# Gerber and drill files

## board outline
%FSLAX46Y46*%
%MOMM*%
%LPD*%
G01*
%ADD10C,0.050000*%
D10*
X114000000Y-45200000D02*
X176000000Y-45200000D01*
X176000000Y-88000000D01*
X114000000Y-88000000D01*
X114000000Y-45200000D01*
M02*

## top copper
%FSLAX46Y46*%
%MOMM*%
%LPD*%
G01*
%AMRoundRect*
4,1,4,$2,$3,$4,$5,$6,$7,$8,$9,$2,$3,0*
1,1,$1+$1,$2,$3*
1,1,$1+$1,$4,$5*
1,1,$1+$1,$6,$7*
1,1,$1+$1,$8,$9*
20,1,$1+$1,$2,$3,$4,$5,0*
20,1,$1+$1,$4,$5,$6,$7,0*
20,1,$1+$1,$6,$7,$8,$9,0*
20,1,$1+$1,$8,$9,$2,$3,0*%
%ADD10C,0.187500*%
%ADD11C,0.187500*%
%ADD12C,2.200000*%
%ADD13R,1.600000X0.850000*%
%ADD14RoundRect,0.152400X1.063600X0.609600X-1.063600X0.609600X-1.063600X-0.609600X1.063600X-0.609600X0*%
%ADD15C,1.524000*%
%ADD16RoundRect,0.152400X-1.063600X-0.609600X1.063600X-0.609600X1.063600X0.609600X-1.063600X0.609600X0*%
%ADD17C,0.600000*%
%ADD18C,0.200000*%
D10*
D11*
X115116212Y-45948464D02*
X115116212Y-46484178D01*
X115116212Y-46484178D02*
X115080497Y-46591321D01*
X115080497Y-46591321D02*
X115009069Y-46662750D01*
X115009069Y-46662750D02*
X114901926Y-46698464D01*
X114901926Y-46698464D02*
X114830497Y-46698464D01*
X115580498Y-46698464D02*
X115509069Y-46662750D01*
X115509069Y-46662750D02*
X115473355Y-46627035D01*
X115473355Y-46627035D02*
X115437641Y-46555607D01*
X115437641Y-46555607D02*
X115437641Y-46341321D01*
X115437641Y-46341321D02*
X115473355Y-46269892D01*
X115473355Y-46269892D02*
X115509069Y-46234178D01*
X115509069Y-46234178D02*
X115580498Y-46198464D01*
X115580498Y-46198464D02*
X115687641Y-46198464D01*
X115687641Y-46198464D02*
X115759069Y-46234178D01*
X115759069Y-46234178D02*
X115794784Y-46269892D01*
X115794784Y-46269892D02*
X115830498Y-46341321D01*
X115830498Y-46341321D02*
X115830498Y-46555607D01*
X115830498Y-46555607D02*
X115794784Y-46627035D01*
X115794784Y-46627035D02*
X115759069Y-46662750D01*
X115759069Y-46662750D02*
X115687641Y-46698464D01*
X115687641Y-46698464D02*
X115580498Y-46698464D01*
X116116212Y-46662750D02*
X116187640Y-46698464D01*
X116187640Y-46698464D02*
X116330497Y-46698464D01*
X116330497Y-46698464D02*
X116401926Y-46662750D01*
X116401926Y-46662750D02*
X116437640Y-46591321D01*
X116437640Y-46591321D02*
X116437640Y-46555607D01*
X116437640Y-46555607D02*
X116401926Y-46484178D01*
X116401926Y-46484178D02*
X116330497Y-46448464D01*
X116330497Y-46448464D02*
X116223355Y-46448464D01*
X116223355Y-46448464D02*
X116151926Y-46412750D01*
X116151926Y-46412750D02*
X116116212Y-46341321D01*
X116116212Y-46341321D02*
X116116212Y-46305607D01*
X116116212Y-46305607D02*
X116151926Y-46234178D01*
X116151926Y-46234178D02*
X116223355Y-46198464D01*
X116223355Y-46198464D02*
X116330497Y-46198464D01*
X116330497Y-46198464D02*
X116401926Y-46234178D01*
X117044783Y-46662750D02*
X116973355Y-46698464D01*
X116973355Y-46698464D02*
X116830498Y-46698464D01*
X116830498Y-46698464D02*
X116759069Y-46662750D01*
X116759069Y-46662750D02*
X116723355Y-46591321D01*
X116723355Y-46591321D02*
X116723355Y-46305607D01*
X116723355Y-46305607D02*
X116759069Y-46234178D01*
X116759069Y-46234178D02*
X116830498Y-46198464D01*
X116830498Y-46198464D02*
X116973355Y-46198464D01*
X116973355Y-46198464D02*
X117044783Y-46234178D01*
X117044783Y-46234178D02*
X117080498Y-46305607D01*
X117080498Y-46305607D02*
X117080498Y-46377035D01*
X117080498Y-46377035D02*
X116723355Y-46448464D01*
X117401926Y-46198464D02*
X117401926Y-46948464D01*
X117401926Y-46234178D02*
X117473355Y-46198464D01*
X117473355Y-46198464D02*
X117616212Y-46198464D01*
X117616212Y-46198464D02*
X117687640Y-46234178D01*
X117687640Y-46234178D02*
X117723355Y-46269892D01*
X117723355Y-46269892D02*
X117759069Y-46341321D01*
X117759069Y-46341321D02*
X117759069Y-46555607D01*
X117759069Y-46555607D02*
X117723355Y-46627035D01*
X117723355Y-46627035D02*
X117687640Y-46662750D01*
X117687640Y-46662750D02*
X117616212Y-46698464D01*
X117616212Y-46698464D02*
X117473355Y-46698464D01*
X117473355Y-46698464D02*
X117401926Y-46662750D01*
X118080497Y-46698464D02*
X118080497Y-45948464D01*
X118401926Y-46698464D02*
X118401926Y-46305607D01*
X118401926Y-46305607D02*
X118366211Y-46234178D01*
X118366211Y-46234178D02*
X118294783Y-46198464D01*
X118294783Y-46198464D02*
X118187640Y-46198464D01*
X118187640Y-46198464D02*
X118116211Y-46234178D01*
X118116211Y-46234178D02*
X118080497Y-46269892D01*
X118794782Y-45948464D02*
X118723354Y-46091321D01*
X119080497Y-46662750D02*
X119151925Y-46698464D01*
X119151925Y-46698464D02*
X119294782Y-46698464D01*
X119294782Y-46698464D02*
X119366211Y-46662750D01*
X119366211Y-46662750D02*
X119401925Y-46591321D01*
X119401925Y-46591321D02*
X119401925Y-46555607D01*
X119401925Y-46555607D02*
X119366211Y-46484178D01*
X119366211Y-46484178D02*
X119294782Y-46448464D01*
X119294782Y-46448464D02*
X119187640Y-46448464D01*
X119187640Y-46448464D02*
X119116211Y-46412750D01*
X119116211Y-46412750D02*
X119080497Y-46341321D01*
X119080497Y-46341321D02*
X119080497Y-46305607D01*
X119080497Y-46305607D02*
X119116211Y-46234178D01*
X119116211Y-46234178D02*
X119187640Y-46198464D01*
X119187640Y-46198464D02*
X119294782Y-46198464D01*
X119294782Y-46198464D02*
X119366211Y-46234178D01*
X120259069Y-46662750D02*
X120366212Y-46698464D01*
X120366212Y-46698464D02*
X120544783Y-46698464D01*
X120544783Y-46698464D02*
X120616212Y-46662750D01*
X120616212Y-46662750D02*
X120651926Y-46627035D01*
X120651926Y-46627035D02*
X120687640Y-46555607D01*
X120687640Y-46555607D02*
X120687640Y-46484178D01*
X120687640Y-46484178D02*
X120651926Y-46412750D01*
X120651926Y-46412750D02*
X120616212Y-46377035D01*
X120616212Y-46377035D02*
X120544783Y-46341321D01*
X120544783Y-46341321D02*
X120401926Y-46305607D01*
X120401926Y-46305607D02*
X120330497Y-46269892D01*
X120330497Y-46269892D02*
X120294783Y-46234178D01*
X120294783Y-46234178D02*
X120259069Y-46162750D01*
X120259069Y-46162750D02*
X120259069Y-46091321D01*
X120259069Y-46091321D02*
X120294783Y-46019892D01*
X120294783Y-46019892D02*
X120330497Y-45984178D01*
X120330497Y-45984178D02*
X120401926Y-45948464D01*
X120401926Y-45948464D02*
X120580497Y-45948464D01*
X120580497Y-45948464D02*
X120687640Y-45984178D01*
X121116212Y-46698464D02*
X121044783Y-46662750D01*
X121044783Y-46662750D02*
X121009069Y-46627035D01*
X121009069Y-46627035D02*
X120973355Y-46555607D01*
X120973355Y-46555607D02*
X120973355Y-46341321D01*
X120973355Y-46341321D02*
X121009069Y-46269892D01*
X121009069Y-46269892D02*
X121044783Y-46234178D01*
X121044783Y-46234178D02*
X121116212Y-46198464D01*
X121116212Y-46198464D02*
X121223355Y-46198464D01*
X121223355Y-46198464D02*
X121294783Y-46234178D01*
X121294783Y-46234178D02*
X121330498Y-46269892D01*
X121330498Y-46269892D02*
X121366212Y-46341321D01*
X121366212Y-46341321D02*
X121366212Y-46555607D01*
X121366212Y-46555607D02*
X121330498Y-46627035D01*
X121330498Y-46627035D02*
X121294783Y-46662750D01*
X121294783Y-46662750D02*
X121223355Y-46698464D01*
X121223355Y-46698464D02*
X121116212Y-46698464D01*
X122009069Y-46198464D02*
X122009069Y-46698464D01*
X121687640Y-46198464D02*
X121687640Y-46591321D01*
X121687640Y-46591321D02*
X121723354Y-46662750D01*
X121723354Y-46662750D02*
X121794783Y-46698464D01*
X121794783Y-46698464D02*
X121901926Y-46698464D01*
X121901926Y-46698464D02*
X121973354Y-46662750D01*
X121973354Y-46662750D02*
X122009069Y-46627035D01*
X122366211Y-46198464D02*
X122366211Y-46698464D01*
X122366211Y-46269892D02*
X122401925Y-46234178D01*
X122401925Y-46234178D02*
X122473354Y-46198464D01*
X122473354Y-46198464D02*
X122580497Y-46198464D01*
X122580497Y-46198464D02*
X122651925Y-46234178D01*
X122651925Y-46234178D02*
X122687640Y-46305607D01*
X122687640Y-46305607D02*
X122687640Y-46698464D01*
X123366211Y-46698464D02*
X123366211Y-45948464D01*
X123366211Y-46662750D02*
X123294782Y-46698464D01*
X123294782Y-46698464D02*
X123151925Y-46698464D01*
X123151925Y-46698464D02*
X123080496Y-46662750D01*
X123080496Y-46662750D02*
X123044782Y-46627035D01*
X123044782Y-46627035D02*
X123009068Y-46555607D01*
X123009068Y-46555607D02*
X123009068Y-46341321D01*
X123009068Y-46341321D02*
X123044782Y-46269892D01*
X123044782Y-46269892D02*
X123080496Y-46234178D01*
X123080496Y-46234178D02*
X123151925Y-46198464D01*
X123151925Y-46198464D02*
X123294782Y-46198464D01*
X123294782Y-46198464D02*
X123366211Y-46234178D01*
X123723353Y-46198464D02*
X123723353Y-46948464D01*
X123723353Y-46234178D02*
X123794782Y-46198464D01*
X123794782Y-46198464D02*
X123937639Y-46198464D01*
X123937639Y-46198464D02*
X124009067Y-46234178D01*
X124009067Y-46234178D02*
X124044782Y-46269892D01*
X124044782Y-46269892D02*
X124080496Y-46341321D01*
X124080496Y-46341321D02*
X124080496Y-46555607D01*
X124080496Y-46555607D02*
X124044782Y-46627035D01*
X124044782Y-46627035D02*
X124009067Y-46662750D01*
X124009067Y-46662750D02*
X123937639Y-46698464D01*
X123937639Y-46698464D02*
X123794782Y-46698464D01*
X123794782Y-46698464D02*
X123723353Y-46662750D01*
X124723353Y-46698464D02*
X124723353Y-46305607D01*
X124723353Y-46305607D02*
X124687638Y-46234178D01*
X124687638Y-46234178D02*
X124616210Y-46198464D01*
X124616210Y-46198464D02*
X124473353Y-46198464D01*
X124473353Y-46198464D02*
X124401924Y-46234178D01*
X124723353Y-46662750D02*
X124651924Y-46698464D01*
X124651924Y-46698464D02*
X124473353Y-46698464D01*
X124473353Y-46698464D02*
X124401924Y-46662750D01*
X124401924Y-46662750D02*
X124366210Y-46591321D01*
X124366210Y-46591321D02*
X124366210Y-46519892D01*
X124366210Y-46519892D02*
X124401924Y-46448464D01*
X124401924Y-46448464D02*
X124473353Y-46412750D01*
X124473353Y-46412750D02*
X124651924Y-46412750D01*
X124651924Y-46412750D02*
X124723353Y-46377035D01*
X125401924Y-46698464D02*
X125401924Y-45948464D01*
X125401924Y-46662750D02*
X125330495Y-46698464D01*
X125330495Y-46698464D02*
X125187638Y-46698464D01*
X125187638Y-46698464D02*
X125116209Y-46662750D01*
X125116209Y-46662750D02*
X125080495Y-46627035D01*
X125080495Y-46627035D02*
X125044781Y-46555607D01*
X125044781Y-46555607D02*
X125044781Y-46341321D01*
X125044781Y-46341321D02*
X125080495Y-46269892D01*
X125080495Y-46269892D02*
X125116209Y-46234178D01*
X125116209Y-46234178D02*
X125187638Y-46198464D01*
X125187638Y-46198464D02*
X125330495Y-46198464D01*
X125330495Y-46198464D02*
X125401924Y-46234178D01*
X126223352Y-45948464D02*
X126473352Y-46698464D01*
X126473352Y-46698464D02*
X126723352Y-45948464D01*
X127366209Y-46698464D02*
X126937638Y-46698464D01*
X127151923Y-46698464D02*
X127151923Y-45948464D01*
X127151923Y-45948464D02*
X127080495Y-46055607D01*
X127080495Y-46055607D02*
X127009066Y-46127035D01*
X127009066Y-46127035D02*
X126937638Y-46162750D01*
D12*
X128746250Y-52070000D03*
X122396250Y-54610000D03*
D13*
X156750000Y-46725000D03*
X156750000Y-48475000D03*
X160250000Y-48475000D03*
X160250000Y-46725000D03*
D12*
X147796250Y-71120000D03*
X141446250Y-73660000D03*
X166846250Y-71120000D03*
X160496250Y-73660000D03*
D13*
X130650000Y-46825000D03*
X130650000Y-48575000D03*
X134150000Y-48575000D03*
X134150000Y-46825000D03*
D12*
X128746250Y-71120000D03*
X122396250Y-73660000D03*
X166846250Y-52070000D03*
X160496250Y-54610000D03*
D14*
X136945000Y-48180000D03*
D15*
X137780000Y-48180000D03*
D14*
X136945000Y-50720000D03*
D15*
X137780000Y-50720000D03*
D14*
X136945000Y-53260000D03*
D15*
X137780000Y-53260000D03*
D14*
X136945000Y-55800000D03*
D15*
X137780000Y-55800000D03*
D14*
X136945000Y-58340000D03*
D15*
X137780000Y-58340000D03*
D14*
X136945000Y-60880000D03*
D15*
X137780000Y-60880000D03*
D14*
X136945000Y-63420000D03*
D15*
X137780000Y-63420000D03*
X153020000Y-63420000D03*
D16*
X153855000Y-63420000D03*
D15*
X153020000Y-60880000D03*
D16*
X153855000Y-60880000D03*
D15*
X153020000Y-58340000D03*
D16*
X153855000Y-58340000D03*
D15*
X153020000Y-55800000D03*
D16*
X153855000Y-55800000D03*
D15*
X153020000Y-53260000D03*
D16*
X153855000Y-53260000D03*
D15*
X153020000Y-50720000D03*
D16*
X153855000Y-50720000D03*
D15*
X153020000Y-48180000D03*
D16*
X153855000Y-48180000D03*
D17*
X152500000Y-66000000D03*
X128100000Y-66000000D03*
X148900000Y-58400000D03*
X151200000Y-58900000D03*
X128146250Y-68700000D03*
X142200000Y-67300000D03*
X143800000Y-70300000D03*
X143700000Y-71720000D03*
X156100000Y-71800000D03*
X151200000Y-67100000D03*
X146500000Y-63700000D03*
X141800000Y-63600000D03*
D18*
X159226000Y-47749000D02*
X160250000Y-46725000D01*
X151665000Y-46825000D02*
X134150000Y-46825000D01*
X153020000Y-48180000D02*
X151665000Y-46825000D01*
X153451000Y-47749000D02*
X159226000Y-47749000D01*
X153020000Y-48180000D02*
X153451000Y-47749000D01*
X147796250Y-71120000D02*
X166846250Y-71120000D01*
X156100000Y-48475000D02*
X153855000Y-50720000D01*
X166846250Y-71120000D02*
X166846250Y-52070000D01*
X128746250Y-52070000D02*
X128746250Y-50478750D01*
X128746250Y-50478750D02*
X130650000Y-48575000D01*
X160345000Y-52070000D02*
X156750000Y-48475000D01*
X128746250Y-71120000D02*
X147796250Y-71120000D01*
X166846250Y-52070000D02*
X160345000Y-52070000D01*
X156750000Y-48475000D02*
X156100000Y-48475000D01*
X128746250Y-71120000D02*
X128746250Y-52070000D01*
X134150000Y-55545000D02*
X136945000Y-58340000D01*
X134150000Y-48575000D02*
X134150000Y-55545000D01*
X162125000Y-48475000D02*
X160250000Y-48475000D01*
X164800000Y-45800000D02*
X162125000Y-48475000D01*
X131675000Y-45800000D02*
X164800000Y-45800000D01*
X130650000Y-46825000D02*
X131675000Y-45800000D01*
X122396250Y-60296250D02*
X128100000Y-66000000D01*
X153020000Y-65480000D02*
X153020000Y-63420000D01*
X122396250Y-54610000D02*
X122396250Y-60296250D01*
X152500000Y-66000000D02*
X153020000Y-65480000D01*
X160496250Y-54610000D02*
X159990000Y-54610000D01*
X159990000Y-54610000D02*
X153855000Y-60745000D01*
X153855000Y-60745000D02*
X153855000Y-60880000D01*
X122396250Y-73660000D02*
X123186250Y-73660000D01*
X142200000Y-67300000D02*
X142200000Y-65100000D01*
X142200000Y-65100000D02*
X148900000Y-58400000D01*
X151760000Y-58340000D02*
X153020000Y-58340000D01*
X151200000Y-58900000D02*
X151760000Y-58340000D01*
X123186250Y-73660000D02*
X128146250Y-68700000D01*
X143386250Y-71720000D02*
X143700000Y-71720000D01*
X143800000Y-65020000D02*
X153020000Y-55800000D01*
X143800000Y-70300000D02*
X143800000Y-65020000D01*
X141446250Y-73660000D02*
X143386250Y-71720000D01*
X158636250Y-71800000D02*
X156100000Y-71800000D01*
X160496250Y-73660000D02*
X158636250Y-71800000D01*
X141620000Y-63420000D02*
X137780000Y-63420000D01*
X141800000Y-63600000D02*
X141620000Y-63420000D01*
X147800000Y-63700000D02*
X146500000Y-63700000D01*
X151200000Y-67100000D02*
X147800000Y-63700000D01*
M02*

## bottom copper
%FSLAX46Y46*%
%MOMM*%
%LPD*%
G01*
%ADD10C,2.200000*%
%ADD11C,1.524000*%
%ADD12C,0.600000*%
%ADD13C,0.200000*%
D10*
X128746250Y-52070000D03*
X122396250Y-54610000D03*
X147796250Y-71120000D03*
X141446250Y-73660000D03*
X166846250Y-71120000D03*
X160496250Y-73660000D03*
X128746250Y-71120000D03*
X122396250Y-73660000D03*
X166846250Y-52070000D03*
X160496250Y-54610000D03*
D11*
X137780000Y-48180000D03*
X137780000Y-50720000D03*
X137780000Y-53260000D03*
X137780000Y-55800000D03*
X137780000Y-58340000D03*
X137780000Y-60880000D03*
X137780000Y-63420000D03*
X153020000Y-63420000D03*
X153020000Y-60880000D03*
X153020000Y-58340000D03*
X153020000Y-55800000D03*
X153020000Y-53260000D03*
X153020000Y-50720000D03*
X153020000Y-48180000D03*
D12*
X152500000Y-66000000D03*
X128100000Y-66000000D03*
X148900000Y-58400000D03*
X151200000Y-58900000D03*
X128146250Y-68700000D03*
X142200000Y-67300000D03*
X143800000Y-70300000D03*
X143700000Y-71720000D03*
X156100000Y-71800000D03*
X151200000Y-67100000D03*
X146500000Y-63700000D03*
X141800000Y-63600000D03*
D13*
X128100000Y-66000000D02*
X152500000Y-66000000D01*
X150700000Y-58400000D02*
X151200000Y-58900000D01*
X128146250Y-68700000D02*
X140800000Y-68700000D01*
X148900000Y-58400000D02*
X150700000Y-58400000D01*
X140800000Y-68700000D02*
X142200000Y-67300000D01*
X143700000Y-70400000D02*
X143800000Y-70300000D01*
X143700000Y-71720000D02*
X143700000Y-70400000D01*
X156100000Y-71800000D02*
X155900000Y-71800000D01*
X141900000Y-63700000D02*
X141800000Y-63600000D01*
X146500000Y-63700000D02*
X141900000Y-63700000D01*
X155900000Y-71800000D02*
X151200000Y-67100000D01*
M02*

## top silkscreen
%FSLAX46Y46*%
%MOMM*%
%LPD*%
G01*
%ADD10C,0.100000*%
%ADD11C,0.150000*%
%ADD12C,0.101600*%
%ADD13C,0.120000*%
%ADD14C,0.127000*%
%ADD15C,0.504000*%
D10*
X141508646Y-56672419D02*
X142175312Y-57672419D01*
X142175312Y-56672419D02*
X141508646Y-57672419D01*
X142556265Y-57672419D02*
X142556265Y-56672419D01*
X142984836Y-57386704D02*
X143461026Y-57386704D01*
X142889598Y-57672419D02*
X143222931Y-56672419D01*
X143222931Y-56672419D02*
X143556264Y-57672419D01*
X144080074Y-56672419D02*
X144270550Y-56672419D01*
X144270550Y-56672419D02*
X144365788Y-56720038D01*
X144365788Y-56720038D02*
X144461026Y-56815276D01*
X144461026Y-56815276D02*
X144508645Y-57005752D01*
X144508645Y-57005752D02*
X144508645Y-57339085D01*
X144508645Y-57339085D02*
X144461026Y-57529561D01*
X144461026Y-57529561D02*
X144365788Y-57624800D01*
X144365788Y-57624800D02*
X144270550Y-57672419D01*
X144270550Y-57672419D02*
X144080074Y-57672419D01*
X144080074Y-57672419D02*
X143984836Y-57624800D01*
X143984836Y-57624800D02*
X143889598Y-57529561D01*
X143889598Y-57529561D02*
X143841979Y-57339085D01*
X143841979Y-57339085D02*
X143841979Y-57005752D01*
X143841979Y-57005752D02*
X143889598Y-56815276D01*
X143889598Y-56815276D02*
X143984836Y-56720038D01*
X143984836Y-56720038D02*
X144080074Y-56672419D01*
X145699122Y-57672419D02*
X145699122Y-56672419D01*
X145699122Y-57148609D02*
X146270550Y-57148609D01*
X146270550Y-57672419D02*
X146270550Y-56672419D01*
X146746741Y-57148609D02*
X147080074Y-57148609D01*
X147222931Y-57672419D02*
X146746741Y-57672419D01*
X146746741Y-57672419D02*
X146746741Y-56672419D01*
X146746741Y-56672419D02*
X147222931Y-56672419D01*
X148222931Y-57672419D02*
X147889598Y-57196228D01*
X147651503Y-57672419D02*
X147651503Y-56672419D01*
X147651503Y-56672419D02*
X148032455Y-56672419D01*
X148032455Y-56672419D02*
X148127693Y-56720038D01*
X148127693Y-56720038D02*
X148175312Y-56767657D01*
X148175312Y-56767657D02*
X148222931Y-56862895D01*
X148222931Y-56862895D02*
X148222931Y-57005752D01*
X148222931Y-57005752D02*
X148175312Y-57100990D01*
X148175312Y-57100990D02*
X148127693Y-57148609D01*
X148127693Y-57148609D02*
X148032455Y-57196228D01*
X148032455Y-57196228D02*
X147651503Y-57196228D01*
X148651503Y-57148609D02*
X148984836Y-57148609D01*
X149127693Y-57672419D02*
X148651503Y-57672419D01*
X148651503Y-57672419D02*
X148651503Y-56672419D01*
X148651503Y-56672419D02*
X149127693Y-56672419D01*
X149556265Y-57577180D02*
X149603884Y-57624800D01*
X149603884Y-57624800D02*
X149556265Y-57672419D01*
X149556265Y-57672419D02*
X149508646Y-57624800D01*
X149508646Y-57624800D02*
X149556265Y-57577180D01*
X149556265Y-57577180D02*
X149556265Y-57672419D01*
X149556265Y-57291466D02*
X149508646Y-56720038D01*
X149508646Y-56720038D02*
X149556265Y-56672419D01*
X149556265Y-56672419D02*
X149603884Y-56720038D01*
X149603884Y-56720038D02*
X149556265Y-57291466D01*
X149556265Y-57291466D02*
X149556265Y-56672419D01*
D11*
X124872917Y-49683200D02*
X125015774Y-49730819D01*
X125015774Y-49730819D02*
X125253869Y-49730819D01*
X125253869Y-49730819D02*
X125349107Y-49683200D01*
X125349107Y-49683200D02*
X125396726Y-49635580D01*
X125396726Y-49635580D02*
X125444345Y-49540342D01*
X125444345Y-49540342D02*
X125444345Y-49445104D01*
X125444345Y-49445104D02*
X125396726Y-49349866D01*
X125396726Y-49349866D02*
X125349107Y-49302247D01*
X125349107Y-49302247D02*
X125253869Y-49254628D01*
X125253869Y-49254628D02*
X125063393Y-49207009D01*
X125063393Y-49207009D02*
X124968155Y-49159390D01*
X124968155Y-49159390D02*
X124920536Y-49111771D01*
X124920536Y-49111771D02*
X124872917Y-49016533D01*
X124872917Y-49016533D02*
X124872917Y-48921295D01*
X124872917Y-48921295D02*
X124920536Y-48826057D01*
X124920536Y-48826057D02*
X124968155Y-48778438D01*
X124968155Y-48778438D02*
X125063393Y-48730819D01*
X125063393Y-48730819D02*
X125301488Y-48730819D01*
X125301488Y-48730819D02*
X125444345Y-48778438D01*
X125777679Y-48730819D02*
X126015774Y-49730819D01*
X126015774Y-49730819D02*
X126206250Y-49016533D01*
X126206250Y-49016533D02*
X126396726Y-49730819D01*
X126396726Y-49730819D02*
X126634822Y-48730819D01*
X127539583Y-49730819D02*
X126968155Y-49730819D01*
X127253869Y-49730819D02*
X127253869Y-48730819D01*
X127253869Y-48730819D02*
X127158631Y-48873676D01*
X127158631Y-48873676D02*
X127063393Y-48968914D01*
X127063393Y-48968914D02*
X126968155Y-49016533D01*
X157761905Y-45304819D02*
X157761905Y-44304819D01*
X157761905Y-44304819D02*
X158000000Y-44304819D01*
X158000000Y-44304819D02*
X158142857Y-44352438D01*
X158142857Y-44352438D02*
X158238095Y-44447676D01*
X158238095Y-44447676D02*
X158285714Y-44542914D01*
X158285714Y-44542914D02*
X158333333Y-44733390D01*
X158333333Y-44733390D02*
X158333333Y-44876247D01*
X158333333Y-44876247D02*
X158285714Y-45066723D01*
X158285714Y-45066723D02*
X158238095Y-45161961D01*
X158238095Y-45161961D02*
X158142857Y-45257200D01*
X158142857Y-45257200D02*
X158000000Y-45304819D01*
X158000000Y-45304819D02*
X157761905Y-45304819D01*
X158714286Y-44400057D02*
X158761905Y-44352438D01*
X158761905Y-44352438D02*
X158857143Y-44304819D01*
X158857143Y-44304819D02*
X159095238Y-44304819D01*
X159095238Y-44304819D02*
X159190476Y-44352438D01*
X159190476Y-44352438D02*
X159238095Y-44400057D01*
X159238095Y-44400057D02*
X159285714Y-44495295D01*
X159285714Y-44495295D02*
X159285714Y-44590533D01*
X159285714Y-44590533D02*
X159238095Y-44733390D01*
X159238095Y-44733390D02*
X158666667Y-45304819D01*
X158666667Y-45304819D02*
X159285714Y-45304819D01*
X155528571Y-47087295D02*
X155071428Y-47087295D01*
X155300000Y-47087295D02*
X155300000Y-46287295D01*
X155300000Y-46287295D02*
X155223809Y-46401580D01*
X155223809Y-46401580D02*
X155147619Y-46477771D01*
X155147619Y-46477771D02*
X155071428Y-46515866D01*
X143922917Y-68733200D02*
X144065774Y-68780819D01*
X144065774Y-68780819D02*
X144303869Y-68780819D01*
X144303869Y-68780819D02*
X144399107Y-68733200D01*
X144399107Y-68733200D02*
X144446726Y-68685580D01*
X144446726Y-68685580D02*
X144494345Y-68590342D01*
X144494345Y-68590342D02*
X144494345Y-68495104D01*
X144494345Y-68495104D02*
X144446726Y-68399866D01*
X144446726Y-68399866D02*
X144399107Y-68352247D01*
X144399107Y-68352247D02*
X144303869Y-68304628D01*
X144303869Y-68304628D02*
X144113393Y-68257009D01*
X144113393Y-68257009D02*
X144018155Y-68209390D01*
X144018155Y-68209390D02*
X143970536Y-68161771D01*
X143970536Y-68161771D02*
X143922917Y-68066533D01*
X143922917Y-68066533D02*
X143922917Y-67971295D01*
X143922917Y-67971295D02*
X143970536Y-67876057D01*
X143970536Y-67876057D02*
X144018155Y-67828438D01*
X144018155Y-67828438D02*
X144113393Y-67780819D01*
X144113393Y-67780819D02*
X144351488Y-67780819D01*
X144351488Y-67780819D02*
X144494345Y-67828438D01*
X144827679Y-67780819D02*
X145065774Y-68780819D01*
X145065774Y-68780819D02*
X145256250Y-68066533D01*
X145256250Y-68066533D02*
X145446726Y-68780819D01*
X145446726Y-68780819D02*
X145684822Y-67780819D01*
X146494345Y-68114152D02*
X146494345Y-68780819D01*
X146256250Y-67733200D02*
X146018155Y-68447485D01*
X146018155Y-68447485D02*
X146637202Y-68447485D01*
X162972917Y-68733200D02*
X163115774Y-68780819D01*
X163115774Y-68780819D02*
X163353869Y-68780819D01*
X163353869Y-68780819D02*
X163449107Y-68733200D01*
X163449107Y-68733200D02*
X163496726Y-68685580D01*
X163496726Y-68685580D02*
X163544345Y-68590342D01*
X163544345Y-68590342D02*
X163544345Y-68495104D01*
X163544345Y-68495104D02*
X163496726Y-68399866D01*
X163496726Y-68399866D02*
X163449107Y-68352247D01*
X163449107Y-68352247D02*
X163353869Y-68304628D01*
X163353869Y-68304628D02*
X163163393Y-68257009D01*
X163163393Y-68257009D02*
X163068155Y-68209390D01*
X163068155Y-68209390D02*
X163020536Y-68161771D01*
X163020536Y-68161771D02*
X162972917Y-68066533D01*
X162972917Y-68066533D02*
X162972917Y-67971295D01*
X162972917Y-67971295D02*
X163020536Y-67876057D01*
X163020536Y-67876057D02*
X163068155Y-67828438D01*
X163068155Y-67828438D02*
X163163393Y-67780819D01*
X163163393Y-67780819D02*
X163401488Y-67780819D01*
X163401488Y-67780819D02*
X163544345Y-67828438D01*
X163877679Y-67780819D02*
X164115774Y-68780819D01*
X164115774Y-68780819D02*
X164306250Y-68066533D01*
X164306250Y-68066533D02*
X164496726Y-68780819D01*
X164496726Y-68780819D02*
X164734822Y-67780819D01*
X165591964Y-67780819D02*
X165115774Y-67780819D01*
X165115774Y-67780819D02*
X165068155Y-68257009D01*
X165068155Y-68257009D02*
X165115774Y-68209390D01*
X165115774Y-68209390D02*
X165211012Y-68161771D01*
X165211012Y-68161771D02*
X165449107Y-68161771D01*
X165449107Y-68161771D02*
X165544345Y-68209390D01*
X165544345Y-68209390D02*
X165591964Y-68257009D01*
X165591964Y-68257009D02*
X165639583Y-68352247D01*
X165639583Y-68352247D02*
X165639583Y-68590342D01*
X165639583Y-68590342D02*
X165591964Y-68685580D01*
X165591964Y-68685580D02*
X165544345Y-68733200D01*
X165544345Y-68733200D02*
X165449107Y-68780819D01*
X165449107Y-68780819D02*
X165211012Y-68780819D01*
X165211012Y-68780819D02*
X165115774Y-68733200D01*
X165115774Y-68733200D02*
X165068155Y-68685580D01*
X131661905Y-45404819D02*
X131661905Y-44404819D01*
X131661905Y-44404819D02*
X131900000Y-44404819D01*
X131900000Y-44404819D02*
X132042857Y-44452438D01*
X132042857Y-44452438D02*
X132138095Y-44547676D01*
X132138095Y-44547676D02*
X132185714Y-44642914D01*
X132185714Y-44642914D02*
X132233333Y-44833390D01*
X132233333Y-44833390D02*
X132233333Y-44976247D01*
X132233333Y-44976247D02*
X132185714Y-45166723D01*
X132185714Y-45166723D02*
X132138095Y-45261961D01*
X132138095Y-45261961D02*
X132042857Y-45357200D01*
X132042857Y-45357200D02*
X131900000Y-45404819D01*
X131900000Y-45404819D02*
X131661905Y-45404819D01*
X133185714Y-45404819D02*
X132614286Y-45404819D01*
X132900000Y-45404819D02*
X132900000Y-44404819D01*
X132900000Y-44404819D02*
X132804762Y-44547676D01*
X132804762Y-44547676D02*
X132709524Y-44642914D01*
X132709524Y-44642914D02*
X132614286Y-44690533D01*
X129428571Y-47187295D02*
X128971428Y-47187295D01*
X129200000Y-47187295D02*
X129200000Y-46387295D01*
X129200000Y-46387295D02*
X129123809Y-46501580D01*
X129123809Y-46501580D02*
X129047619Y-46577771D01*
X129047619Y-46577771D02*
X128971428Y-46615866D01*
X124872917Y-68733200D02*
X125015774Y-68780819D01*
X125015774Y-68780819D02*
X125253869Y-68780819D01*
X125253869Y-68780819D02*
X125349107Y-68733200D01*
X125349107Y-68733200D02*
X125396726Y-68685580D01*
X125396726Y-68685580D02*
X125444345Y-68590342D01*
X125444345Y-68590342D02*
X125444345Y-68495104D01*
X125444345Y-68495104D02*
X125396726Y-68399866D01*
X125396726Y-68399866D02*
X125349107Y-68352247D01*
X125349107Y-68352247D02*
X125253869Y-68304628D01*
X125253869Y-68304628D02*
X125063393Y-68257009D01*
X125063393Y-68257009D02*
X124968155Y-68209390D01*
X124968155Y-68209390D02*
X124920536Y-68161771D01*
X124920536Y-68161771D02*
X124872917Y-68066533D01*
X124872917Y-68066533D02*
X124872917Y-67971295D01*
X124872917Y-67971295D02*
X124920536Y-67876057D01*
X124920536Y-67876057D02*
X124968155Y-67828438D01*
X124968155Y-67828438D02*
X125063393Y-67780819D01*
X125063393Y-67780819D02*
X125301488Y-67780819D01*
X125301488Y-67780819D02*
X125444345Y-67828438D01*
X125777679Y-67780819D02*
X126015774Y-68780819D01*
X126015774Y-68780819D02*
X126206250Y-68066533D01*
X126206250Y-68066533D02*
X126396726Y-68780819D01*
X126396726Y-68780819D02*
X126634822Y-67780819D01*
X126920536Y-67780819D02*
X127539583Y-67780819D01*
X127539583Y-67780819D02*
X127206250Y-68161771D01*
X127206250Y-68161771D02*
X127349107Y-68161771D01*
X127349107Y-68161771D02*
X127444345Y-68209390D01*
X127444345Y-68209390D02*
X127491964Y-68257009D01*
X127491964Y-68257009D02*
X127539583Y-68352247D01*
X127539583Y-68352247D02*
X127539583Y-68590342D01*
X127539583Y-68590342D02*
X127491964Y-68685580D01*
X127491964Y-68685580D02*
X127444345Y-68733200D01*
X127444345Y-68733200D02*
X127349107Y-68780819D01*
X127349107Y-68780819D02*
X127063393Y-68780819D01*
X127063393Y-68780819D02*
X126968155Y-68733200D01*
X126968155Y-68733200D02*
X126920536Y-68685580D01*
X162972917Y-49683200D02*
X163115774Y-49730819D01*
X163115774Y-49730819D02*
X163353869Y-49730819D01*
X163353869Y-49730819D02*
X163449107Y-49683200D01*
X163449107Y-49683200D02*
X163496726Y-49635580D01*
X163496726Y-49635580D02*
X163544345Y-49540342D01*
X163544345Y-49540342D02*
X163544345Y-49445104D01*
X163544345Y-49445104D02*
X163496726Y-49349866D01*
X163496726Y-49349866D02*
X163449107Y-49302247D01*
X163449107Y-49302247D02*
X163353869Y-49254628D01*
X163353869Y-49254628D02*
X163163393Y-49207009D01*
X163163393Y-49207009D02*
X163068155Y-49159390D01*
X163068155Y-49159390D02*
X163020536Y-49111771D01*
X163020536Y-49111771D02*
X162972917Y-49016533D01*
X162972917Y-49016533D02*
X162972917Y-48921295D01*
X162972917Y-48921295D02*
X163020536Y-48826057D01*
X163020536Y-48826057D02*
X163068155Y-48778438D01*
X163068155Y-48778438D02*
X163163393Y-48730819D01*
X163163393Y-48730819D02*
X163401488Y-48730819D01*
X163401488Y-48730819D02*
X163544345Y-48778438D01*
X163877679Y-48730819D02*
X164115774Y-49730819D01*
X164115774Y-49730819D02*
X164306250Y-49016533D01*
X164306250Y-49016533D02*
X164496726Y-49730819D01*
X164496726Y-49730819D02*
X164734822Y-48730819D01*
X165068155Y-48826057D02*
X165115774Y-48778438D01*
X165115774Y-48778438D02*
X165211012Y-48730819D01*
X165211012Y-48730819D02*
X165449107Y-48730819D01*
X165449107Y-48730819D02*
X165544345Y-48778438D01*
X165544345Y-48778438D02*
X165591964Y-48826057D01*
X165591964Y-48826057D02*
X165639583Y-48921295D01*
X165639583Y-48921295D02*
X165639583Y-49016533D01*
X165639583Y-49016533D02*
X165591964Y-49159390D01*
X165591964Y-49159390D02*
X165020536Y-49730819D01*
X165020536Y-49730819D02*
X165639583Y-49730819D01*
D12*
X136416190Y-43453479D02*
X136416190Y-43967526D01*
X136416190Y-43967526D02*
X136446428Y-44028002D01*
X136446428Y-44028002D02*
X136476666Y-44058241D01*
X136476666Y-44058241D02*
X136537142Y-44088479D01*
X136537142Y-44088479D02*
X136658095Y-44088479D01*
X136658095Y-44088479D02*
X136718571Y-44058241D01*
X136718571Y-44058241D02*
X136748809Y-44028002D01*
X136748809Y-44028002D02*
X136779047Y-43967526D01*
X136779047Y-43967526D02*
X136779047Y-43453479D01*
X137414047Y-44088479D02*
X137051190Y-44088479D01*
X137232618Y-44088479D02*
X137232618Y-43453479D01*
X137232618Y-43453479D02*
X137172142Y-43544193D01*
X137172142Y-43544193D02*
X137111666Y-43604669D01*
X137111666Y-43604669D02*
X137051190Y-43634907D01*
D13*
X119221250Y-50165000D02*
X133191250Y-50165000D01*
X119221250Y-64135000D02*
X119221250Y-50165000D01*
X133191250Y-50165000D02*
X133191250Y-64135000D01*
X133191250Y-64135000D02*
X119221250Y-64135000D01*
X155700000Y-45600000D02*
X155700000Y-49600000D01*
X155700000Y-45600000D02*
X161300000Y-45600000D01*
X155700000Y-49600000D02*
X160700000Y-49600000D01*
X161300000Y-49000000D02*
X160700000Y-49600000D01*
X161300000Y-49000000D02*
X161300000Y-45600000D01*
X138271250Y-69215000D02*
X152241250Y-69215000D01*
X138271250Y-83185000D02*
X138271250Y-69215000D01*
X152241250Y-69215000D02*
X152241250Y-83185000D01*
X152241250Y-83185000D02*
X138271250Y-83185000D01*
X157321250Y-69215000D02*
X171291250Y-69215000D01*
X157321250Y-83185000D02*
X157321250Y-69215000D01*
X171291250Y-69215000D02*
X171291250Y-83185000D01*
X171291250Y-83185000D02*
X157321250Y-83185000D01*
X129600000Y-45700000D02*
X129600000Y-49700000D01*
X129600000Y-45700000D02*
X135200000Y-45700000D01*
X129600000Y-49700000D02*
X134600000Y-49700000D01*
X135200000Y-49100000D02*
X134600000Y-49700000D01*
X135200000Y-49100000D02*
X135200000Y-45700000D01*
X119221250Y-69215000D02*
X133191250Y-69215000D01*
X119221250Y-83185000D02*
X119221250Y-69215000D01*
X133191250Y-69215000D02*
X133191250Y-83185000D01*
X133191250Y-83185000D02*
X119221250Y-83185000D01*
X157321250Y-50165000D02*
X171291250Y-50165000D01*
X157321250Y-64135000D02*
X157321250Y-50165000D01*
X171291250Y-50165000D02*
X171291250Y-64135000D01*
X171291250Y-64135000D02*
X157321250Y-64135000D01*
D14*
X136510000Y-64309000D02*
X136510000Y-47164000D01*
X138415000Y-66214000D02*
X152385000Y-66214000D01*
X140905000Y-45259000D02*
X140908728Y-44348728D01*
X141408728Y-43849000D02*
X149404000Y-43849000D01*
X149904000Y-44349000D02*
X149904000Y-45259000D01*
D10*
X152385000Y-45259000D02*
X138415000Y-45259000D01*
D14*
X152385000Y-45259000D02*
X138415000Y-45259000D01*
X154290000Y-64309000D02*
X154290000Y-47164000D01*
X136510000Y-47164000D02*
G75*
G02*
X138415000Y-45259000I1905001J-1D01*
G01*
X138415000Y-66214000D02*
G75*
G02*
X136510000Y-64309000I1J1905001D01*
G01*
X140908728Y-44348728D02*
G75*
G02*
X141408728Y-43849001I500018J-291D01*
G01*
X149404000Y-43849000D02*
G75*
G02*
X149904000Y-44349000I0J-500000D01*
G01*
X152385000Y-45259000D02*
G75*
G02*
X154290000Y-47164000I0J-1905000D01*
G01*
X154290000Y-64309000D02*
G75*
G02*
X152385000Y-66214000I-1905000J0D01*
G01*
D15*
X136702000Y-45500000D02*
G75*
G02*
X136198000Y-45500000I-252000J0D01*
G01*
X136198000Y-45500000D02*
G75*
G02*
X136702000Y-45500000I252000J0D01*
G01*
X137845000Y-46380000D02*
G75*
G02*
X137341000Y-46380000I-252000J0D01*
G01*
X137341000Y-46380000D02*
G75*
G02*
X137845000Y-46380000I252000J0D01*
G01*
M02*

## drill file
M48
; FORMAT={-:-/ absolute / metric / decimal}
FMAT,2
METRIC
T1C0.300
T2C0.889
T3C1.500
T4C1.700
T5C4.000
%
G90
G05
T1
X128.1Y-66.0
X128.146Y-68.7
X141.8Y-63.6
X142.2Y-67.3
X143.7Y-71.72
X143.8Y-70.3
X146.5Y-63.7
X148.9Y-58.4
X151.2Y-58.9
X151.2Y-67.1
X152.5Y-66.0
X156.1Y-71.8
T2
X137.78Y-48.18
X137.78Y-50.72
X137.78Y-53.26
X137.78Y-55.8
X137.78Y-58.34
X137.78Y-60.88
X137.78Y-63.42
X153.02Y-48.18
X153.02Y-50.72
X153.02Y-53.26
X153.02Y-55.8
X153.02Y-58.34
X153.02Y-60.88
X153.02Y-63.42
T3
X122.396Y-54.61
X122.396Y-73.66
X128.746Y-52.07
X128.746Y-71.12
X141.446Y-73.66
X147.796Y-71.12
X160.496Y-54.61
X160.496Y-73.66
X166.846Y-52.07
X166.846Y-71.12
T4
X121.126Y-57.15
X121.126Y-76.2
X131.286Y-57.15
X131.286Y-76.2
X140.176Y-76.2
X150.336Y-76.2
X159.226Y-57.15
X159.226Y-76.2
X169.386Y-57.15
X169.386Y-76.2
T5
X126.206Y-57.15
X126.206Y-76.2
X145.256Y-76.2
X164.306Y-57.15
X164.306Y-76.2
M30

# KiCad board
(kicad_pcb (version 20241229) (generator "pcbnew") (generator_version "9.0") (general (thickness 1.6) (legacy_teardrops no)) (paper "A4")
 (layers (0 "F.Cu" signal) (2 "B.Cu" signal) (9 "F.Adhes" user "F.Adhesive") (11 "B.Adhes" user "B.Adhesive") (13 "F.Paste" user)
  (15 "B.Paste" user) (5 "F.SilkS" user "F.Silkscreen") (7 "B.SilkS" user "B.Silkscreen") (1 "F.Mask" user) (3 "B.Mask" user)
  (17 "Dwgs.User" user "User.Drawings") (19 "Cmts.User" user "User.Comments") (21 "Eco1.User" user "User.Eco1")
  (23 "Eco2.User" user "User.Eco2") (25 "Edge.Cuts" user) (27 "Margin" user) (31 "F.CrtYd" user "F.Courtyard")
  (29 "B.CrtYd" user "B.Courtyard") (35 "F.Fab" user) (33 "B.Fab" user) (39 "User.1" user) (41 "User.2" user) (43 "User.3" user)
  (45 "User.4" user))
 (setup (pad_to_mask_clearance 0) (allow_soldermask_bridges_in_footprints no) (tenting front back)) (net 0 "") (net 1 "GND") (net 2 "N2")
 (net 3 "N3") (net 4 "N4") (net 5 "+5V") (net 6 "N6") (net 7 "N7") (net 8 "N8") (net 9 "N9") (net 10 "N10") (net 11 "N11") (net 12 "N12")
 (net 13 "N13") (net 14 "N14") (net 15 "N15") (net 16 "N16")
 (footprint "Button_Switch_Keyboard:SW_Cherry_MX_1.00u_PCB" (layer "F.Cu") (at 128.74625 52.07)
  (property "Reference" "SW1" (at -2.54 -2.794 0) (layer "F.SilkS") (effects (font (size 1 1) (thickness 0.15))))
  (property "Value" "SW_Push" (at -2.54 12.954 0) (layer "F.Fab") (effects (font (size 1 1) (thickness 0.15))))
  (fp_line (start -9.525 -1.905) (end 4.445 -1.905) (stroke (width 0.12) (type solid)) (layer "F.SilkS"))
  (fp_line (start -9.525 12.065) (end -9.525 -1.905) (stroke (width 0.12) (type solid)) (layer "F.SilkS"))
  (fp_line (start 4.445 -1.905) (end 4.445 12.065) (stroke (width 0.12) (type solid)) (layer "F.SilkS"))
  (fp_line (start 4.445 12.065) (end -9.525 12.065) (stroke (width 0.12) (type solid)) (layer "F.SilkS"))
  (pad "" np_thru_hole circle (at -7.62 5.08) (size 1.7 1.7) (drill 1.7) (layers "*.Cu" "*.Mask"))
  (pad "" np_thru_hole circle (at -2.54 5.08) (size 4 4) (drill 4) (layers "*.Cu" "*.Mask"))
  (pad "" np_thru_hole circle (at 2.54 5.08) (size 1.7 1.7) (drill 1.7) (layers "*.Cu" "*.Mask"))
  (pad "1" thru_hole circle (at 0 0) (size 2.2 2.2) (drill 1.5) (layers "*.Cu" "*.Mask") (remove_unused_layers no) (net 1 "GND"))
  (pad "2" thru_hole circle (at -6.35 2.54) (size 2.2 2.2) (drill 1.5) (layers "*.Cu" "*.Mask") (remove_unused_layers no) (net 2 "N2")))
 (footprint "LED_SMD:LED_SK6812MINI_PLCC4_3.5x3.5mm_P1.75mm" (layer "F.Cu") (at 158.5 47.6)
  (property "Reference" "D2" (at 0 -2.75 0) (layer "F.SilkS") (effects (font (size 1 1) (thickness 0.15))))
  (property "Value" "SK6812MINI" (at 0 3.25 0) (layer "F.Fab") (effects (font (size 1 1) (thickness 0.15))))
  (fp_line (start -2.8 -2) (end -2.8 2) (stroke (width 0.12) (type default)) (layer "F.SilkS"))
  (fp_line (start -2.8 -2) (end 2.8 -2) (stroke (width 0.12) (type solid)) (layer "F.SilkS"))
  (fp_line (start -2.8 2) (end 2.2 2) (stroke (width 0.12) (type solid)) (layer "F.SilkS"))
  (fp_line (start 2.8 1.4) (end 2.2 2) (stroke (width 0.12) (type default)) (layer "F.SilkS"))
  (fp_line (start 2.8 1.4) (end 2.8 -2) (stroke (width 0.12) (type solid)) (layer "F.SilkS"))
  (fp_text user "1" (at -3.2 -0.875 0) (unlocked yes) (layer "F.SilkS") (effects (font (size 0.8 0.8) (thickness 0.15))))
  (pad "1" smd rect (at -1.75 -0.875) (size 1.6 0.85) (layers "F.Cu" "F.Mask" "F.Paste") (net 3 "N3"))
  (pad "2" smd rect (at -1.75 0.875) (size 1.6 0.85) (layers "F.Cu" "F.Mask" "F.Paste") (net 1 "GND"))
  (pad "3" smd rect (at 1.75 0.875) (size 1.6 0.85) (layers "F.Cu" "F.Mask" "F.Paste") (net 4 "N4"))
  (pad "4" smd rect (at 1.75 -0.875) (size 1.6 0.85) (layers "F.Cu" "F.Mask" "F.Paste") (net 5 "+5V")))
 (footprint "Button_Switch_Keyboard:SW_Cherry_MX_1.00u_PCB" (layer "F.Cu") (at 147.79625 71.12)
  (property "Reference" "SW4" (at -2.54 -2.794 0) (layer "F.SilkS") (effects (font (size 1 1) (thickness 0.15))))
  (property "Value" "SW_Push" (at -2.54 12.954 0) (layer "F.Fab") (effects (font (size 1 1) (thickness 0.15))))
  (fp_line (start -9.525 -1.905) (end 4.445 -1.905) (stroke (width 0.12) (type solid)) (layer "F.SilkS"))
  (fp_line (start -9.525 12.065) (end -9.525 -1.905) (stroke (width 0.12) (type solid)) (layer "F.SilkS"))
  (fp_line (start 4.445 -1.905) (end 4.445 12.065) (stroke (width 0.12) (type solid)) (layer "F.SilkS"))
  (fp_line (start 4.445 12.065) (end -9.525 12.065) (stroke (width 0.12) (type solid)) (layer "F.SilkS"))
  (pad "" np_thru_hole circle (at -7.62 5.08) (size 1.7 1.7) (drill 1.7) (layers "*.Cu" "*.Mask"))
  (pad "" np_thru_hole circle (at -2.54 5.08) (size 4 4) (drill 4) (layers "*.Cu" "*.Mask"))
  (pad "" np_thru_hole circle (at 2.54 5.08) (size 1.7 1.7) (drill 1.7) (layers "*.Cu" "*.Mask"))
  (pad "1" thru_hole circle (at 0 0) (size 2.2 2.2) (drill 1.5) (layers "*.Cu" "*.Mask") (remove_unused_layers no) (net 1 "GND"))
  (pad "2" thru_hole circle (at -6.35 2.54) (size 2.2 2.2) (drill 1.5) (layers "*.Cu" "*.Mask") (remove_unused_layers no) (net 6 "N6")))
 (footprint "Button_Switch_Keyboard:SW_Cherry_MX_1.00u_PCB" (layer "F.Cu") (at 166.84625 71.12)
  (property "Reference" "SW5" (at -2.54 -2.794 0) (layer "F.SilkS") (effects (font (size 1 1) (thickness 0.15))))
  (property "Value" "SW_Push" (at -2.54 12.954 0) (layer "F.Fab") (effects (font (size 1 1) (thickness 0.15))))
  (fp_line (start -9.525 -1.905) (end 4.445 -1.905) (stroke (width 0.12) (type solid)) (layer "F.SilkS"))
  (fp_line (start -9.525 12.065) (end -9.525 -1.905) (stroke (width 0.12) (type solid)) (layer "F.SilkS"))
  (fp_line (start 4.445 -1.905) (end 4.445 12.065) (stroke (width 0.12) (type solid)) (layer "F.SilkS"))
  (fp_line (start 4.445 12.065) (end -9.525 12.065) (stroke (width 0.12) (type solid)) (layer "F.SilkS"))
  (pad "" np_thru_hole circle (at -7.62 5.08) (size 1.7 1.7) (drill 1.7) (layers "*.Cu" "*.Mask"))
  (pad "" np_thru_hole circle (at -2.54 5.08) (size 4 4) (drill 4) (layers "*.Cu" "*.Mask"))
  (pad "" np_thru_hole circle (at 2.54 5.08) (size 1.7 1.7) (drill 1.7) (layers "*.Cu" "*.Mask"))
  (pad "1" thru_hole circle (at 0 0) (size 2.2 2.2) (drill 1.5) (layers "*.Cu" "*.Mask") (remove_unused_layers no) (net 1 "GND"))
  (pad "2" thru_hole circle (at -6.35 2.54) (size 2.2 2.2) (drill 1.5) (layers "*.Cu" "*.Mask") (remove_unused_layers no) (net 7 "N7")))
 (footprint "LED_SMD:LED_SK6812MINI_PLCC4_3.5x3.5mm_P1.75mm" (layer "F.Cu") (at 132.4 47.7)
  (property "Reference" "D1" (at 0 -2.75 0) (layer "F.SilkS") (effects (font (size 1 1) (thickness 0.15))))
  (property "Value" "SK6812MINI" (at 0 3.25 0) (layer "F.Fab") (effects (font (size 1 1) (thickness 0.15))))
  (fp_line (start -2.8 -2) (end -2.8 2) (stroke (width 0.12) (type default)) (layer "F.SilkS"))
  (fp_line (start -2.8 -2) (end 2.8 -2) (stroke (width 0.12) (type solid)) (layer "F.SilkS"))
  (fp_line (start -2.8 2) (end 2.2 2) (stroke (width 0.12) (type solid)) (layer "F.SilkS"))
  (fp_line (start 2.8 1.4) (end 2.2 2) (stroke (width 0.12) (type default)) (layer "F.SilkS"))
  (fp_line (start 2.8 1.4) (end 2.8 -2) (stroke (width 0.12) (type solid)) (layer "F.SilkS"))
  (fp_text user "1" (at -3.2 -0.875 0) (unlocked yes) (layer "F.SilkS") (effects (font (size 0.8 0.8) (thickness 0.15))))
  (pad "1" smd rect (at -1.75 -0.875) (size 1.6 0.85) (layers "F.Cu" "F.Mask" "F.Paste") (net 4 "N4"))
  (pad "2" smd rect (at -1.75 0.875) (size 1.6 0.85) (layers "F.Cu" "F.Mask" "F.Paste") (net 1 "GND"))
  (pad "3" smd rect (at 1.75 0.875) (size 1.6 0.85) (layers "F.Cu" "F.Mask" "F.Paste") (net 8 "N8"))
  (pad "4" smd rect (at 1.75 -0.875) (size 1.6 0.85) (layers "F.Cu" "F.Mask" "F.Paste") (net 5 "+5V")))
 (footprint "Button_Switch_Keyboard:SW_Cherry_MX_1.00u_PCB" (layer "F.Cu") (at 128.74625 71.12)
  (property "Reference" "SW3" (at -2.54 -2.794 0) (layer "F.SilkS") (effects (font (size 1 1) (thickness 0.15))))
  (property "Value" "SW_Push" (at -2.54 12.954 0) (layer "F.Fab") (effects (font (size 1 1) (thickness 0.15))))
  (fp_line (start -9.525 -1.905) (end 4.445 -1.905) (stroke (width 0.12) (type solid)) (layer "F.SilkS"))
  (fp_line (start -9.525 12.065) (end -9.525 -1.905) (stroke (width 0.12) (type solid)) (layer "F.SilkS"))
  (fp_line (start 4.445 -1.905) (end 4.445 12.065) (stroke (width 0.12) (type solid)) (layer "F.SilkS"))
  (fp_line (start 4.445 12.065) (end -9.525 12.065) (stroke (width 0.12) (type solid)) (layer "F.SilkS"))
  (pad "" np_thru_hole circle (at -7.62 5.08) (size 1.7 1.7) (drill 1.7) (layers "*.Cu" "*.Mask"))
  (pad "" np_thru_hole circle (at -2.54 5.08) (size 4 4) (drill 4) (layers "*.Cu" "*.Mask"))
  (pad "" np_thru_hole circle (at 2.54 5.08) (size 1.7 1.7) (drill 1.7) (layers "*.Cu" "*.Mask"))
  (pad "1" thru_hole circle (at 0 0) (size 2.2 2.2) (drill 1.5) (layers "*.Cu" "*.Mask") (remove_unused_layers no) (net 1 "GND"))
  (pad "2" thru_hole circle (at -6.35 2.54) (size 2.2 2.2) (drill 1.5) (layers "*.Cu" "*.Mask") (remove_unused_layers no) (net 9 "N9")))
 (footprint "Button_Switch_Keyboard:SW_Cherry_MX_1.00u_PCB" (layer "F.Cu") (at 166.84625 52.07)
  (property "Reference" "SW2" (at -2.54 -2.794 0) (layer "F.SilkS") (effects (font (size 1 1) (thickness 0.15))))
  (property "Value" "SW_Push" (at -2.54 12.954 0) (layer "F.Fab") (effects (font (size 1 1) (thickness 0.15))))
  (fp_line (start -9.525 -1.905) (end 4.445 -1.905) (stroke (width 0.12) (type solid)) (layer "F.SilkS"))
  (fp_line (start -9.525 12.065) (end -9.525 -1.905) (stroke (width 0.12) (type solid)) (layer "F.SilkS"))
  (fp_line (start 4.445 -1.905) (end 4.445 12.065) (stroke (width 0.12) (type solid)) (layer "F.SilkS"))
  (fp_line (start 4.445 12.065) (end -9.525 12.065) (stroke (width 0.12) (type solid)) (layer "F.SilkS"))
  (pad "" np_thru_hole circle (at -7.62 5.08) (size 1.7 1.7) (drill 1.7) (layers "*.Cu" "*.Mask"))
  (pad "" np_thru_hole circle (at -2.54 5.08) (size 4 4) (drill 4) (layers "*.Cu" "*.Mask"))
  (pad "" np_thru_hole circle (at 2.54 5.08) (size 1.7 1.7) (drill 1.7) (layers "*.Cu" "*.Mask"))
  (pad "1" thru_hole circle (at 0 0) (size 2.2 2.2) (drill 1.5) (layers "*.Cu" "*.Mask") (remove_unused_layers no) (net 1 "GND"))
  (pad "2" thru_hole circle (at -6.35 2.54) (size 2.2 2.2) (drill 1.5) (layers "*.Cu" "*.Mask") (remove_unused_layers no) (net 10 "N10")))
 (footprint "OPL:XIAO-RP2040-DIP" (layer "F.Cu") (at 145.4 55.8)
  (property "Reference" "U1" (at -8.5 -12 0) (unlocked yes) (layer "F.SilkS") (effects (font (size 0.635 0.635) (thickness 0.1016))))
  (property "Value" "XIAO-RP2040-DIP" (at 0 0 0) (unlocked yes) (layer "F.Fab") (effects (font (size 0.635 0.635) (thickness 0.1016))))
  (fp_line (start -8.89 8.509) (end -8.89 -8.636) (stroke (width 0.127) (type solid)) (layer "F.SilkS"))
  (fp_line (start -6.985 10.414) (end 6.985 10.414) (stroke (width 0.127) (type solid)) (layer "F.SilkS"))
  (fp_line (start -4.495 -10.541) (end -4.491272 -11.451272) (stroke (width 0.127) (type solid)) (layer "F.SilkS"))
  (fp_line (start -3.991272 -11.951) (end 4.004 -11.951) (stroke (width 0.127) (type solid)) (layer "F.SilkS"))
  (fp_line (start 4.504 -11.451) (end 4.504 -10.541) (stroke (width 0.127) (type solid)) (layer "F.SilkS"))
  (fp_line (start 6.985 -10.541) (end -6.985 -10.541) (stroke (width 0.1) (type solid)) (layer "F.SilkS"))
  (fp_line (start 6.985 -10.541) (end -6.985 -10.541) (stroke (width 0.127) (type solid)) (layer "F.SilkS"))
  (fp_line (start 8.89 8.509) (end 8.89 -8.636) (stroke (width 0.127) (type solid)) (layer "F.SilkS"))
  (fp_arc (start -8.89 -8.636) (mid -8.332038 -9.983038) (end -6.985 -10.541) (stroke (width 0.127) (type solid)) (layer "F.SilkS"))
  (fp_arc (start -6.985 10.414) (mid -8.332038 9.856038) (end -8.89 8.509) (stroke (width 0.127) (type solid)) (layer "F.SilkS"))
  (fp_arc (start -4.491272 -11.451272) (mid -4.344728 -11.80464) (end -3.991272 -11.951) (stroke (width 0.127) (type default))
   (layer "F.SilkS"))
  (fp_arc (start 4.004 -11.951) (mid 4.357553 -11.804553) (end 4.504 -11.451) (stroke (width 0.127) (type default)) (layer "F.SilkS"))
  (fp_arc (start 6.985 -10.541) (mid 8.332038 -9.983038) (end 8.89 -8.636) (stroke (width 0.127) (type solid)) (layer "F.SilkS"))
  (fp_arc (start 8.89 8.509) (mid 8.332038 9.856038) (end 6.985 10.414) (stroke (width 0.127) (type solid)) (layer "F.SilkS"))
  (fp_circle (center -8.95 -10.3) (end -8.95 -10.554) (stroke (width 0.5) (type solid)) (fill yes) (layer "F.SilkS"))
  (fp_circle (center -7.807 -9.42) (end -7.807 -9.674) (stroke (width 0.5) (type solid)) (fill yes) (layer "F.SilkS"))
  (pad "1" smd roundrect (at -8.455 -7.62 180) (size 2.432 1.524) (layers "F.Cu" "F.Mask") (roundrect_rratio 0.1) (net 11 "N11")
   (thermal_bridge_angle 45))
  (pad "1" thru_hole circle (at -7.62 -7.62 180) (size 1.524 1.524) (drill 0.889) (layers "*.Cu" "*.Mask") (remove_unused_layers no)
   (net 11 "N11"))
  (pad "2" smd roundrect (at -8.455 -5.08 180) (size 2.432 1.524) (layers "F.Cu" "F.Mask") (roundrect_rratio 0.1) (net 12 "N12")
   (thermal_bridge_angle 45))
  (pad "2" thru_hole circle (at -7.62 -5.08 180) (size 1.524 1.524) (drill 0.889) (layers "*.Cu" "*.Mask") (remove_unused_layers no)
   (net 12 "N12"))
  (pad "3" smd roundrect (at -8.455 -2.54 180) (size 2.432 1.524) (layers "F.Cu" "F.Mask") (roundrect_rratio 0.1) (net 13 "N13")
   (thermal_bridge_angle 45))
  (pad "3" thru_hole circle (at -7.62 -2.54 180) (size 1.524 1.524) (drill 0.889) (layers "*.Cu" "*.Mask") (remove_unused_layers no)
   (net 13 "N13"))
  (pad "4" smd roundrect (at -8.455 0 180) (size 2.432 1.524) (layers "F.Cu" "F.Mask") (roundrect_rratio 0.1) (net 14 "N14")
   (thermal_bridge_angle 45))
  (pad "4" thru_hole circle (at -7.62 0 180) (size 1.524 1.524) (drill 0.889) (layers "*.Cu" "*.Mask") (remove_unused_layers no)
   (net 14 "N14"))
  (pad "5" smd roundrect (at -8.455 2.54 180) (size 2.432 1.524) (layers "F.Cu" "F.Mask") (roundrect_rratio 0.1) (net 8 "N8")
   (thermal_bridge_angle 45))
  (pad "5" thru_hole circle (at -7.62 2.54 180) (size 1.524 1.524) (drill 0.889) (layers "*.Cu" "*.Mask") (remove_unused_layers no)
   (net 8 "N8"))
  (pad "6" smd roundrect (at -8.455 5.08 180) (size 2.432 1.524) (layers "F.Cu" "F.Mask") (roundrect_rratio 0.1) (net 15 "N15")
   (thermal_bridge_angle 45))
  (pad "6" thru_hole circle (at -7.62 5.08 180) (size 1.524 1.524) (drill 0.889) (layers "*.Cu" "*.Mask") (remove_unused_layers no)
   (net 15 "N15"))
  (pad "7" smd roundrect (at -8.455 7.62 180) (size 2.432 1.524) (layers "F.Cu" "F.Mask") (roundrect_rratio 0.1) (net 7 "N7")
   (thermal_bridge_angle 45))
  (pad "7" thru_hole circle (at -7.62 7.62 180) (size 1.524 1.524) (drill 0.889) (layers "*.Cu" "*.Mask") (remove_unused_layers no)
   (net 7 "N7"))
  (pad "8" thru_hole circle (at 7.62 7.62) (size 1.524 1.524) (drill 0.889) (layers "*.Cu" "*.Mask") (remove_unused_layers no) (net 2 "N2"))
  (pad "8" smd roundrect (at 8.455 7.62) (size 2.432 1.524) (layers "F.Cu" "F.Mask") (roundrect_rratio 0.1) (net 2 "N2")
   (thermal_bridge_angle 45))
  (pad "9" thru_hole circle (at 7.62 5.08) (size 1.524 1.524) (drill 0.889) (layers "*.Cu" "*.Mask") (remove_unused_layers no)
   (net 10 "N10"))
  (pad "9" smd roundrect (at 8.455 5.08) (size 2.432 1.524) (layers "F.Cu" "F.Mask") (roundrect_rratio 0.1) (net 10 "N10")
   (thermal_bridge_angle 45))
  (pad "10" thru_hole circle (at 7.62 2.54) (size 1.524 1.524) (drill 0.889) (layers "*.Cu" "*.Mask") (remove_unused_layers no) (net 9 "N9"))
  (pad "10" smd roundrect (at 8.455 2.54) (size 2.432 1.524) (layers "F.Cu" "F.Mask") (roundrect_rratio 0.1) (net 9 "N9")
   (thermal_bridge_angle 45))
  (pad "11" thru_hole circle (at 7.62 0) (size 1.524 1.524) (drill 0.889) (layers "*.Cu" "*.Mask") (remove_unused_layers no) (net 6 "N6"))
  (pad "11" smd roundrect (at 8.455 0) (size 2.432 1.524) (layers "F.Cu" "F.Mask") (roundrect_rratio 0.1) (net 6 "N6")
   (thermal_bridge_angle 45))
  (pad "12" thru_hole circle (at 7.62 -2.54) (size 1.524 1.524) (drill 0.889) (layers "*.Cu" "*.Mask") (remove_unused_layers no)
   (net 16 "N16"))
  (pad "12" smd roundrect (at 8.455 -2.54) (size 2.432 1.524) (layers "F.Cu" "F.Mask") (roundrect_rratio 0.1) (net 16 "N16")
   (thermal_bridge_angle 45))
  (pad "13" thru_hole circle (at 7.62 -5.08) (size 1.524 1.524) (drill 0.889) (layers "*.Cu" "*.Mask") (remove_unused_layers no)
   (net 1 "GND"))
  (pad "13" smd roundrect (at 8.455 -5.08) (size 2.432 1.524) (layers "F.Cu" "F.Mask") (roundrect_rratio 0.1) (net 1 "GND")
   (thermal_bridge_angle 45))
  (pad "14" thru_hole circle (at 7.62 -7.62) (size 1.524 1.524) (drill 0.889) (layers "*.Cu" "*.Mask") (remove_unused_layers no)
   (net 5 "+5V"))
  (pad "14" smd roundrect (at 8.455 -7.62) (size 2.432 1.524) (layers "F.Cu" "F.Mask") (roundrect_rratio 0.1) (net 5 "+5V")
   (thermal_bridge_angle 45)))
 (gr_rect (start 114 45.2) (end 176 88) (stroke (width 0.05) (type default)) (fill no) (layer "Edge.Cuts"))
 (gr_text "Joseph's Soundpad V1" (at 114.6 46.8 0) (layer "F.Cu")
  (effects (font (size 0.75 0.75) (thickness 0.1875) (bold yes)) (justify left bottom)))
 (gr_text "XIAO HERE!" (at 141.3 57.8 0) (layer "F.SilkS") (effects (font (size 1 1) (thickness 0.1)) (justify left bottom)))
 (segment (start 159.226 47.749) (end 160.25 46.725) (width 0.2) (layer "F.Cu") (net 5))
 (segment (start 151.665 46.825) (end 134.15 46.825) (width 0.2) (layer "F.Cu") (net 5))
 (segment (start 153.02 48.18) (end 151.665 46.825) (width 0.2) (layer "F.Cu") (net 5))
 (segment (start 153.451 47.749) (end 159.226 47.749) (width 0.2) (layer "F.Cu") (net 5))
 (segment (start 153.02 48.18) (end 153.451 47.749) (width 0.2) (layer "F.Cu") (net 5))
 (segment (start 147.79625 71.12) (end 166.84625 71.12) (width 0.2) (layer "F.Cu") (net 1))
 (segment (start 156.1 48.475) (end 153.855 50.72) (width 0.2) (layer "F.Cu") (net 1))
 (segment (start 166.84625 71.12) (end 166.84625 52.07) (width 0.2) (layer "F.Cu") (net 1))
 (segment (start 128.74625 52.07) (end 128.74625 50.47875) (width 0.2) (layer "F.Cu") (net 1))
 (segment (start 128.74625 50.47875) (end 130.65 48.575) (width 0.2) (layer "F.Cu") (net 1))
 (segment (start 160.345 52.07) (end 156.75 48.475) (width 0.2) (layer "F.Cu") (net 1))
 (segment (start 128.74625 71.12) (end 147.79625 71.12) (width 0.2) (layer "F.Cu") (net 1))
 (segment (start 166.84625 52.07) (end 160.345 52.07) (width 0.2) (layer "F.Cu") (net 1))
 (segment (start 156.75 48.475) (end 156.1 48.475) (width 0.2) (layer "F.Cu") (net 1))
 (segment (start 128.74625 71.12) (end 128.74625 52.07) (width 0.2) (layer "F.Cu") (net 1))
 (segment (start 134.15 55.545) (end 136.945 58.34) (width 0.2) (layer "F.Cu") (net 8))
 (segment (start 134.15 48.575) (end 134.15 55.545) (width 0.2) (layer "F.Cu") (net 8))
 (segment (start 162.125 48.475) (end 160.25 48.475) (width 0.2) (layer "F.Cu") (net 4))
 (segment (start 164.8 45.8) (end 162.125 48.475) (width 0.2) (layer "F.Cu") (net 4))
 (segment (start 131.675 45.8) (end 164.8 45.8) (width 0.2) (layer "F.Cu") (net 4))
 (segment (start 130.65 46.825) (end 131.675 45.8) (width 0.2) (layer "F.Cu") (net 4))
 (segment (start 122.39625 60.29625) (end 128.1 66) (width 0.2) (layer "F.Cu") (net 2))
 (segment (start 153.02 65.48) (end 153.02 63.42) (width 0.2) (layer "F.Cu") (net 2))
 (segment (start 122.39625 54.61) (end 122.39625 60.29625) (width 0.2) (layer "F.Cu") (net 2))
 (segment (start 152.5 66) (end 153.02 65.48) (width 0.2) (layer "F.Cu") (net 2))
 (via (at 152.5 66) (size 0.6) (drill 0.3) (layers "F.Cu" "B.Cu") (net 2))
 (via (at 128.1 66) (size 0.6) (drill 0.3) (layers "F.Cu" "B.Cu") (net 2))
 (segment (start 128.1 66) (end 152.5 66) (width 0.2) (layer "B.Cu") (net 2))
 (segment (start 160.49625 54.61) (end 159.99 54.61) (width 0.2) (layer "F.Cu") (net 10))
 (segment (start 159.99 54.61) (end 153.855 60.745) (width 0.2) (layer "F.Cu") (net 10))
 (segment (start 153.855 60.745) (end 153.855 60.88) (width 0.2) (layer "F.Cu") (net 10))
 (segment (start 122.39625 73.66) (end 123.18625 73.66) (width 0.2) (layer "F.Cu") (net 9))
 (segment (start 142.2 67.3) (end 142.2 65.1) (width 0.2) (layer "F.Cu") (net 9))
 (segment (start 142.2 65.1) (end 148.9 58.4) (width 0.2) (layer "F.Cu") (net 9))
 (segment (start 151.76 58.34) (end 153.02 58.34) (width 0.2) (layer "F.Cu") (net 9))
 (segment (start 151.2 58.9) (end 151.76 58.34) (width 0.2) (layer "F.Cu") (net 9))
 (segment (start 123.18625 73.66) (end 128.14625 68.7) (width 0.2) (layer "F.Cu") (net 9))
 (via (at 148.9 58.4) (size 0.6) (drill 0.3) (layers "F.Cu" "B.Cu") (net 9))
 (via (at 151.2 58.9) (size 0.6) (drill 0.3) (layers "F.Cu" "B.Cu") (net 9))
 (via (at 128.14625 68.7) (size 0.6) (drill 0.3) (layers "F.Cu" "B.Cu") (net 9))
 (via (at 142.2 67.3) (size 0.6) (drill 0.3) (layers "F.Cu" "B.Cu") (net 9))
 (segment (start 150.7 58.4) (end 151.2 58.9) (width 0.2) (layer "B.Cu") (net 9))
 (segment (start 128.14625 68.7) (end 140.8 68.7) (width 0.2) (layer "B.Cu") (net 9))
 (segment (start 148.9 58.4) (end 150.7 58.4) (width 0.2) (layer "B.Cu") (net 9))
 (segment (start 140.8 68.7) (end 142.2 67.3) (width 0.2) (layer "B.Cu") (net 9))
 (segment (start 143.38625 71.72) (end 143.7 71.72) (width 0.2) (layer "F.Cu") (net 6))
 (segment (start 143.8 65.02) (end 153.02 55.8) (width 0.2) (layer "F.Cu") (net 6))
 (segment (start 143.8 70.3) (end 143.8 65.02) (width 0.2) (layer "F.Cu") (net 6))
 (segment (start 141.44625 73.66) (end 143.38625 71.72) (width 0.2) (layer "F.Cu") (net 6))
 (via (at 143.8 70.3) (size 0.6) (drill 0.3) (layers "F.Cu" "B.Cu") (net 6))
 (via (at 143.7 71.72) (size 0.6) (drill 0.3) (layers "F.Cu" "B.Cu") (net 6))
 (segment (start 143.7 70.4) (end 143.8 70.3) (width 0.2) (layer "B.Cu") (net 6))
 (segment (start 143.7 71.72) (end 143.7 70.4) (width 0.2) (layer "B.Cu") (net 6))
 (segment (start 158.63625 71.8) (end 156.1 71.8) (width 0.2) (layer "F.Cu") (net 7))
 (segment (start 160.49625 73.66) (end 158.63625 71.8) (width 0.2) (layer "F.Cu") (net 7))
 (segment (start 141.62 63.42) (end 137.78 63.42) (width 0.2) (layer "F.Cu") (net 7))
 (segment (start 141.8 63.6) (end 141.62 63.42) (width 0.2) (layer "F.Cu") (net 7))
 (segment (start 147.8 63.7) (end 146.5 63.7) (width 0.2) (layer "F.Cu") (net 7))
 (segment (start 151.2 67.1) (end 147.8 63.7) (width 0.2) (layer "F.Cu") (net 7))
 (via (at 156.1 71.8) (size 0.6) (drill 0.3) (layers "F.Cu" "B.Cu") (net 7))
 (via (at 151.2 67.1) (size 0.6) (drill 0.3) (layers "F.Cu" "B.Cu") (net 7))
 (via (at 146.5 63.7) (size 0.6) (drill 0.3) (layers "F.Cu" "B.Cu") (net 7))
 (via (at 141.8 63.6) (size 0.6) (drill 0.3) (layers "F.Cu" "B.Cu") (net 7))
 (segment (start 156.1 71.8) (end 155.9 71.8) (width 0.2) (layer "B.Cu") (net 7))
 (segment (start 141.9 63.7) (end 141.8 63.6) (width 0.2) (layer "B.Cu") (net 7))
 (segment (start 146.5 63.7) (end 141.9 63.7) (width 0.2) (layer "B.Cu") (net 7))
 (segment (start 155.9 71.8) (end 151.2 67.1) (width 0.2) (layer "B.Cu") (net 7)))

